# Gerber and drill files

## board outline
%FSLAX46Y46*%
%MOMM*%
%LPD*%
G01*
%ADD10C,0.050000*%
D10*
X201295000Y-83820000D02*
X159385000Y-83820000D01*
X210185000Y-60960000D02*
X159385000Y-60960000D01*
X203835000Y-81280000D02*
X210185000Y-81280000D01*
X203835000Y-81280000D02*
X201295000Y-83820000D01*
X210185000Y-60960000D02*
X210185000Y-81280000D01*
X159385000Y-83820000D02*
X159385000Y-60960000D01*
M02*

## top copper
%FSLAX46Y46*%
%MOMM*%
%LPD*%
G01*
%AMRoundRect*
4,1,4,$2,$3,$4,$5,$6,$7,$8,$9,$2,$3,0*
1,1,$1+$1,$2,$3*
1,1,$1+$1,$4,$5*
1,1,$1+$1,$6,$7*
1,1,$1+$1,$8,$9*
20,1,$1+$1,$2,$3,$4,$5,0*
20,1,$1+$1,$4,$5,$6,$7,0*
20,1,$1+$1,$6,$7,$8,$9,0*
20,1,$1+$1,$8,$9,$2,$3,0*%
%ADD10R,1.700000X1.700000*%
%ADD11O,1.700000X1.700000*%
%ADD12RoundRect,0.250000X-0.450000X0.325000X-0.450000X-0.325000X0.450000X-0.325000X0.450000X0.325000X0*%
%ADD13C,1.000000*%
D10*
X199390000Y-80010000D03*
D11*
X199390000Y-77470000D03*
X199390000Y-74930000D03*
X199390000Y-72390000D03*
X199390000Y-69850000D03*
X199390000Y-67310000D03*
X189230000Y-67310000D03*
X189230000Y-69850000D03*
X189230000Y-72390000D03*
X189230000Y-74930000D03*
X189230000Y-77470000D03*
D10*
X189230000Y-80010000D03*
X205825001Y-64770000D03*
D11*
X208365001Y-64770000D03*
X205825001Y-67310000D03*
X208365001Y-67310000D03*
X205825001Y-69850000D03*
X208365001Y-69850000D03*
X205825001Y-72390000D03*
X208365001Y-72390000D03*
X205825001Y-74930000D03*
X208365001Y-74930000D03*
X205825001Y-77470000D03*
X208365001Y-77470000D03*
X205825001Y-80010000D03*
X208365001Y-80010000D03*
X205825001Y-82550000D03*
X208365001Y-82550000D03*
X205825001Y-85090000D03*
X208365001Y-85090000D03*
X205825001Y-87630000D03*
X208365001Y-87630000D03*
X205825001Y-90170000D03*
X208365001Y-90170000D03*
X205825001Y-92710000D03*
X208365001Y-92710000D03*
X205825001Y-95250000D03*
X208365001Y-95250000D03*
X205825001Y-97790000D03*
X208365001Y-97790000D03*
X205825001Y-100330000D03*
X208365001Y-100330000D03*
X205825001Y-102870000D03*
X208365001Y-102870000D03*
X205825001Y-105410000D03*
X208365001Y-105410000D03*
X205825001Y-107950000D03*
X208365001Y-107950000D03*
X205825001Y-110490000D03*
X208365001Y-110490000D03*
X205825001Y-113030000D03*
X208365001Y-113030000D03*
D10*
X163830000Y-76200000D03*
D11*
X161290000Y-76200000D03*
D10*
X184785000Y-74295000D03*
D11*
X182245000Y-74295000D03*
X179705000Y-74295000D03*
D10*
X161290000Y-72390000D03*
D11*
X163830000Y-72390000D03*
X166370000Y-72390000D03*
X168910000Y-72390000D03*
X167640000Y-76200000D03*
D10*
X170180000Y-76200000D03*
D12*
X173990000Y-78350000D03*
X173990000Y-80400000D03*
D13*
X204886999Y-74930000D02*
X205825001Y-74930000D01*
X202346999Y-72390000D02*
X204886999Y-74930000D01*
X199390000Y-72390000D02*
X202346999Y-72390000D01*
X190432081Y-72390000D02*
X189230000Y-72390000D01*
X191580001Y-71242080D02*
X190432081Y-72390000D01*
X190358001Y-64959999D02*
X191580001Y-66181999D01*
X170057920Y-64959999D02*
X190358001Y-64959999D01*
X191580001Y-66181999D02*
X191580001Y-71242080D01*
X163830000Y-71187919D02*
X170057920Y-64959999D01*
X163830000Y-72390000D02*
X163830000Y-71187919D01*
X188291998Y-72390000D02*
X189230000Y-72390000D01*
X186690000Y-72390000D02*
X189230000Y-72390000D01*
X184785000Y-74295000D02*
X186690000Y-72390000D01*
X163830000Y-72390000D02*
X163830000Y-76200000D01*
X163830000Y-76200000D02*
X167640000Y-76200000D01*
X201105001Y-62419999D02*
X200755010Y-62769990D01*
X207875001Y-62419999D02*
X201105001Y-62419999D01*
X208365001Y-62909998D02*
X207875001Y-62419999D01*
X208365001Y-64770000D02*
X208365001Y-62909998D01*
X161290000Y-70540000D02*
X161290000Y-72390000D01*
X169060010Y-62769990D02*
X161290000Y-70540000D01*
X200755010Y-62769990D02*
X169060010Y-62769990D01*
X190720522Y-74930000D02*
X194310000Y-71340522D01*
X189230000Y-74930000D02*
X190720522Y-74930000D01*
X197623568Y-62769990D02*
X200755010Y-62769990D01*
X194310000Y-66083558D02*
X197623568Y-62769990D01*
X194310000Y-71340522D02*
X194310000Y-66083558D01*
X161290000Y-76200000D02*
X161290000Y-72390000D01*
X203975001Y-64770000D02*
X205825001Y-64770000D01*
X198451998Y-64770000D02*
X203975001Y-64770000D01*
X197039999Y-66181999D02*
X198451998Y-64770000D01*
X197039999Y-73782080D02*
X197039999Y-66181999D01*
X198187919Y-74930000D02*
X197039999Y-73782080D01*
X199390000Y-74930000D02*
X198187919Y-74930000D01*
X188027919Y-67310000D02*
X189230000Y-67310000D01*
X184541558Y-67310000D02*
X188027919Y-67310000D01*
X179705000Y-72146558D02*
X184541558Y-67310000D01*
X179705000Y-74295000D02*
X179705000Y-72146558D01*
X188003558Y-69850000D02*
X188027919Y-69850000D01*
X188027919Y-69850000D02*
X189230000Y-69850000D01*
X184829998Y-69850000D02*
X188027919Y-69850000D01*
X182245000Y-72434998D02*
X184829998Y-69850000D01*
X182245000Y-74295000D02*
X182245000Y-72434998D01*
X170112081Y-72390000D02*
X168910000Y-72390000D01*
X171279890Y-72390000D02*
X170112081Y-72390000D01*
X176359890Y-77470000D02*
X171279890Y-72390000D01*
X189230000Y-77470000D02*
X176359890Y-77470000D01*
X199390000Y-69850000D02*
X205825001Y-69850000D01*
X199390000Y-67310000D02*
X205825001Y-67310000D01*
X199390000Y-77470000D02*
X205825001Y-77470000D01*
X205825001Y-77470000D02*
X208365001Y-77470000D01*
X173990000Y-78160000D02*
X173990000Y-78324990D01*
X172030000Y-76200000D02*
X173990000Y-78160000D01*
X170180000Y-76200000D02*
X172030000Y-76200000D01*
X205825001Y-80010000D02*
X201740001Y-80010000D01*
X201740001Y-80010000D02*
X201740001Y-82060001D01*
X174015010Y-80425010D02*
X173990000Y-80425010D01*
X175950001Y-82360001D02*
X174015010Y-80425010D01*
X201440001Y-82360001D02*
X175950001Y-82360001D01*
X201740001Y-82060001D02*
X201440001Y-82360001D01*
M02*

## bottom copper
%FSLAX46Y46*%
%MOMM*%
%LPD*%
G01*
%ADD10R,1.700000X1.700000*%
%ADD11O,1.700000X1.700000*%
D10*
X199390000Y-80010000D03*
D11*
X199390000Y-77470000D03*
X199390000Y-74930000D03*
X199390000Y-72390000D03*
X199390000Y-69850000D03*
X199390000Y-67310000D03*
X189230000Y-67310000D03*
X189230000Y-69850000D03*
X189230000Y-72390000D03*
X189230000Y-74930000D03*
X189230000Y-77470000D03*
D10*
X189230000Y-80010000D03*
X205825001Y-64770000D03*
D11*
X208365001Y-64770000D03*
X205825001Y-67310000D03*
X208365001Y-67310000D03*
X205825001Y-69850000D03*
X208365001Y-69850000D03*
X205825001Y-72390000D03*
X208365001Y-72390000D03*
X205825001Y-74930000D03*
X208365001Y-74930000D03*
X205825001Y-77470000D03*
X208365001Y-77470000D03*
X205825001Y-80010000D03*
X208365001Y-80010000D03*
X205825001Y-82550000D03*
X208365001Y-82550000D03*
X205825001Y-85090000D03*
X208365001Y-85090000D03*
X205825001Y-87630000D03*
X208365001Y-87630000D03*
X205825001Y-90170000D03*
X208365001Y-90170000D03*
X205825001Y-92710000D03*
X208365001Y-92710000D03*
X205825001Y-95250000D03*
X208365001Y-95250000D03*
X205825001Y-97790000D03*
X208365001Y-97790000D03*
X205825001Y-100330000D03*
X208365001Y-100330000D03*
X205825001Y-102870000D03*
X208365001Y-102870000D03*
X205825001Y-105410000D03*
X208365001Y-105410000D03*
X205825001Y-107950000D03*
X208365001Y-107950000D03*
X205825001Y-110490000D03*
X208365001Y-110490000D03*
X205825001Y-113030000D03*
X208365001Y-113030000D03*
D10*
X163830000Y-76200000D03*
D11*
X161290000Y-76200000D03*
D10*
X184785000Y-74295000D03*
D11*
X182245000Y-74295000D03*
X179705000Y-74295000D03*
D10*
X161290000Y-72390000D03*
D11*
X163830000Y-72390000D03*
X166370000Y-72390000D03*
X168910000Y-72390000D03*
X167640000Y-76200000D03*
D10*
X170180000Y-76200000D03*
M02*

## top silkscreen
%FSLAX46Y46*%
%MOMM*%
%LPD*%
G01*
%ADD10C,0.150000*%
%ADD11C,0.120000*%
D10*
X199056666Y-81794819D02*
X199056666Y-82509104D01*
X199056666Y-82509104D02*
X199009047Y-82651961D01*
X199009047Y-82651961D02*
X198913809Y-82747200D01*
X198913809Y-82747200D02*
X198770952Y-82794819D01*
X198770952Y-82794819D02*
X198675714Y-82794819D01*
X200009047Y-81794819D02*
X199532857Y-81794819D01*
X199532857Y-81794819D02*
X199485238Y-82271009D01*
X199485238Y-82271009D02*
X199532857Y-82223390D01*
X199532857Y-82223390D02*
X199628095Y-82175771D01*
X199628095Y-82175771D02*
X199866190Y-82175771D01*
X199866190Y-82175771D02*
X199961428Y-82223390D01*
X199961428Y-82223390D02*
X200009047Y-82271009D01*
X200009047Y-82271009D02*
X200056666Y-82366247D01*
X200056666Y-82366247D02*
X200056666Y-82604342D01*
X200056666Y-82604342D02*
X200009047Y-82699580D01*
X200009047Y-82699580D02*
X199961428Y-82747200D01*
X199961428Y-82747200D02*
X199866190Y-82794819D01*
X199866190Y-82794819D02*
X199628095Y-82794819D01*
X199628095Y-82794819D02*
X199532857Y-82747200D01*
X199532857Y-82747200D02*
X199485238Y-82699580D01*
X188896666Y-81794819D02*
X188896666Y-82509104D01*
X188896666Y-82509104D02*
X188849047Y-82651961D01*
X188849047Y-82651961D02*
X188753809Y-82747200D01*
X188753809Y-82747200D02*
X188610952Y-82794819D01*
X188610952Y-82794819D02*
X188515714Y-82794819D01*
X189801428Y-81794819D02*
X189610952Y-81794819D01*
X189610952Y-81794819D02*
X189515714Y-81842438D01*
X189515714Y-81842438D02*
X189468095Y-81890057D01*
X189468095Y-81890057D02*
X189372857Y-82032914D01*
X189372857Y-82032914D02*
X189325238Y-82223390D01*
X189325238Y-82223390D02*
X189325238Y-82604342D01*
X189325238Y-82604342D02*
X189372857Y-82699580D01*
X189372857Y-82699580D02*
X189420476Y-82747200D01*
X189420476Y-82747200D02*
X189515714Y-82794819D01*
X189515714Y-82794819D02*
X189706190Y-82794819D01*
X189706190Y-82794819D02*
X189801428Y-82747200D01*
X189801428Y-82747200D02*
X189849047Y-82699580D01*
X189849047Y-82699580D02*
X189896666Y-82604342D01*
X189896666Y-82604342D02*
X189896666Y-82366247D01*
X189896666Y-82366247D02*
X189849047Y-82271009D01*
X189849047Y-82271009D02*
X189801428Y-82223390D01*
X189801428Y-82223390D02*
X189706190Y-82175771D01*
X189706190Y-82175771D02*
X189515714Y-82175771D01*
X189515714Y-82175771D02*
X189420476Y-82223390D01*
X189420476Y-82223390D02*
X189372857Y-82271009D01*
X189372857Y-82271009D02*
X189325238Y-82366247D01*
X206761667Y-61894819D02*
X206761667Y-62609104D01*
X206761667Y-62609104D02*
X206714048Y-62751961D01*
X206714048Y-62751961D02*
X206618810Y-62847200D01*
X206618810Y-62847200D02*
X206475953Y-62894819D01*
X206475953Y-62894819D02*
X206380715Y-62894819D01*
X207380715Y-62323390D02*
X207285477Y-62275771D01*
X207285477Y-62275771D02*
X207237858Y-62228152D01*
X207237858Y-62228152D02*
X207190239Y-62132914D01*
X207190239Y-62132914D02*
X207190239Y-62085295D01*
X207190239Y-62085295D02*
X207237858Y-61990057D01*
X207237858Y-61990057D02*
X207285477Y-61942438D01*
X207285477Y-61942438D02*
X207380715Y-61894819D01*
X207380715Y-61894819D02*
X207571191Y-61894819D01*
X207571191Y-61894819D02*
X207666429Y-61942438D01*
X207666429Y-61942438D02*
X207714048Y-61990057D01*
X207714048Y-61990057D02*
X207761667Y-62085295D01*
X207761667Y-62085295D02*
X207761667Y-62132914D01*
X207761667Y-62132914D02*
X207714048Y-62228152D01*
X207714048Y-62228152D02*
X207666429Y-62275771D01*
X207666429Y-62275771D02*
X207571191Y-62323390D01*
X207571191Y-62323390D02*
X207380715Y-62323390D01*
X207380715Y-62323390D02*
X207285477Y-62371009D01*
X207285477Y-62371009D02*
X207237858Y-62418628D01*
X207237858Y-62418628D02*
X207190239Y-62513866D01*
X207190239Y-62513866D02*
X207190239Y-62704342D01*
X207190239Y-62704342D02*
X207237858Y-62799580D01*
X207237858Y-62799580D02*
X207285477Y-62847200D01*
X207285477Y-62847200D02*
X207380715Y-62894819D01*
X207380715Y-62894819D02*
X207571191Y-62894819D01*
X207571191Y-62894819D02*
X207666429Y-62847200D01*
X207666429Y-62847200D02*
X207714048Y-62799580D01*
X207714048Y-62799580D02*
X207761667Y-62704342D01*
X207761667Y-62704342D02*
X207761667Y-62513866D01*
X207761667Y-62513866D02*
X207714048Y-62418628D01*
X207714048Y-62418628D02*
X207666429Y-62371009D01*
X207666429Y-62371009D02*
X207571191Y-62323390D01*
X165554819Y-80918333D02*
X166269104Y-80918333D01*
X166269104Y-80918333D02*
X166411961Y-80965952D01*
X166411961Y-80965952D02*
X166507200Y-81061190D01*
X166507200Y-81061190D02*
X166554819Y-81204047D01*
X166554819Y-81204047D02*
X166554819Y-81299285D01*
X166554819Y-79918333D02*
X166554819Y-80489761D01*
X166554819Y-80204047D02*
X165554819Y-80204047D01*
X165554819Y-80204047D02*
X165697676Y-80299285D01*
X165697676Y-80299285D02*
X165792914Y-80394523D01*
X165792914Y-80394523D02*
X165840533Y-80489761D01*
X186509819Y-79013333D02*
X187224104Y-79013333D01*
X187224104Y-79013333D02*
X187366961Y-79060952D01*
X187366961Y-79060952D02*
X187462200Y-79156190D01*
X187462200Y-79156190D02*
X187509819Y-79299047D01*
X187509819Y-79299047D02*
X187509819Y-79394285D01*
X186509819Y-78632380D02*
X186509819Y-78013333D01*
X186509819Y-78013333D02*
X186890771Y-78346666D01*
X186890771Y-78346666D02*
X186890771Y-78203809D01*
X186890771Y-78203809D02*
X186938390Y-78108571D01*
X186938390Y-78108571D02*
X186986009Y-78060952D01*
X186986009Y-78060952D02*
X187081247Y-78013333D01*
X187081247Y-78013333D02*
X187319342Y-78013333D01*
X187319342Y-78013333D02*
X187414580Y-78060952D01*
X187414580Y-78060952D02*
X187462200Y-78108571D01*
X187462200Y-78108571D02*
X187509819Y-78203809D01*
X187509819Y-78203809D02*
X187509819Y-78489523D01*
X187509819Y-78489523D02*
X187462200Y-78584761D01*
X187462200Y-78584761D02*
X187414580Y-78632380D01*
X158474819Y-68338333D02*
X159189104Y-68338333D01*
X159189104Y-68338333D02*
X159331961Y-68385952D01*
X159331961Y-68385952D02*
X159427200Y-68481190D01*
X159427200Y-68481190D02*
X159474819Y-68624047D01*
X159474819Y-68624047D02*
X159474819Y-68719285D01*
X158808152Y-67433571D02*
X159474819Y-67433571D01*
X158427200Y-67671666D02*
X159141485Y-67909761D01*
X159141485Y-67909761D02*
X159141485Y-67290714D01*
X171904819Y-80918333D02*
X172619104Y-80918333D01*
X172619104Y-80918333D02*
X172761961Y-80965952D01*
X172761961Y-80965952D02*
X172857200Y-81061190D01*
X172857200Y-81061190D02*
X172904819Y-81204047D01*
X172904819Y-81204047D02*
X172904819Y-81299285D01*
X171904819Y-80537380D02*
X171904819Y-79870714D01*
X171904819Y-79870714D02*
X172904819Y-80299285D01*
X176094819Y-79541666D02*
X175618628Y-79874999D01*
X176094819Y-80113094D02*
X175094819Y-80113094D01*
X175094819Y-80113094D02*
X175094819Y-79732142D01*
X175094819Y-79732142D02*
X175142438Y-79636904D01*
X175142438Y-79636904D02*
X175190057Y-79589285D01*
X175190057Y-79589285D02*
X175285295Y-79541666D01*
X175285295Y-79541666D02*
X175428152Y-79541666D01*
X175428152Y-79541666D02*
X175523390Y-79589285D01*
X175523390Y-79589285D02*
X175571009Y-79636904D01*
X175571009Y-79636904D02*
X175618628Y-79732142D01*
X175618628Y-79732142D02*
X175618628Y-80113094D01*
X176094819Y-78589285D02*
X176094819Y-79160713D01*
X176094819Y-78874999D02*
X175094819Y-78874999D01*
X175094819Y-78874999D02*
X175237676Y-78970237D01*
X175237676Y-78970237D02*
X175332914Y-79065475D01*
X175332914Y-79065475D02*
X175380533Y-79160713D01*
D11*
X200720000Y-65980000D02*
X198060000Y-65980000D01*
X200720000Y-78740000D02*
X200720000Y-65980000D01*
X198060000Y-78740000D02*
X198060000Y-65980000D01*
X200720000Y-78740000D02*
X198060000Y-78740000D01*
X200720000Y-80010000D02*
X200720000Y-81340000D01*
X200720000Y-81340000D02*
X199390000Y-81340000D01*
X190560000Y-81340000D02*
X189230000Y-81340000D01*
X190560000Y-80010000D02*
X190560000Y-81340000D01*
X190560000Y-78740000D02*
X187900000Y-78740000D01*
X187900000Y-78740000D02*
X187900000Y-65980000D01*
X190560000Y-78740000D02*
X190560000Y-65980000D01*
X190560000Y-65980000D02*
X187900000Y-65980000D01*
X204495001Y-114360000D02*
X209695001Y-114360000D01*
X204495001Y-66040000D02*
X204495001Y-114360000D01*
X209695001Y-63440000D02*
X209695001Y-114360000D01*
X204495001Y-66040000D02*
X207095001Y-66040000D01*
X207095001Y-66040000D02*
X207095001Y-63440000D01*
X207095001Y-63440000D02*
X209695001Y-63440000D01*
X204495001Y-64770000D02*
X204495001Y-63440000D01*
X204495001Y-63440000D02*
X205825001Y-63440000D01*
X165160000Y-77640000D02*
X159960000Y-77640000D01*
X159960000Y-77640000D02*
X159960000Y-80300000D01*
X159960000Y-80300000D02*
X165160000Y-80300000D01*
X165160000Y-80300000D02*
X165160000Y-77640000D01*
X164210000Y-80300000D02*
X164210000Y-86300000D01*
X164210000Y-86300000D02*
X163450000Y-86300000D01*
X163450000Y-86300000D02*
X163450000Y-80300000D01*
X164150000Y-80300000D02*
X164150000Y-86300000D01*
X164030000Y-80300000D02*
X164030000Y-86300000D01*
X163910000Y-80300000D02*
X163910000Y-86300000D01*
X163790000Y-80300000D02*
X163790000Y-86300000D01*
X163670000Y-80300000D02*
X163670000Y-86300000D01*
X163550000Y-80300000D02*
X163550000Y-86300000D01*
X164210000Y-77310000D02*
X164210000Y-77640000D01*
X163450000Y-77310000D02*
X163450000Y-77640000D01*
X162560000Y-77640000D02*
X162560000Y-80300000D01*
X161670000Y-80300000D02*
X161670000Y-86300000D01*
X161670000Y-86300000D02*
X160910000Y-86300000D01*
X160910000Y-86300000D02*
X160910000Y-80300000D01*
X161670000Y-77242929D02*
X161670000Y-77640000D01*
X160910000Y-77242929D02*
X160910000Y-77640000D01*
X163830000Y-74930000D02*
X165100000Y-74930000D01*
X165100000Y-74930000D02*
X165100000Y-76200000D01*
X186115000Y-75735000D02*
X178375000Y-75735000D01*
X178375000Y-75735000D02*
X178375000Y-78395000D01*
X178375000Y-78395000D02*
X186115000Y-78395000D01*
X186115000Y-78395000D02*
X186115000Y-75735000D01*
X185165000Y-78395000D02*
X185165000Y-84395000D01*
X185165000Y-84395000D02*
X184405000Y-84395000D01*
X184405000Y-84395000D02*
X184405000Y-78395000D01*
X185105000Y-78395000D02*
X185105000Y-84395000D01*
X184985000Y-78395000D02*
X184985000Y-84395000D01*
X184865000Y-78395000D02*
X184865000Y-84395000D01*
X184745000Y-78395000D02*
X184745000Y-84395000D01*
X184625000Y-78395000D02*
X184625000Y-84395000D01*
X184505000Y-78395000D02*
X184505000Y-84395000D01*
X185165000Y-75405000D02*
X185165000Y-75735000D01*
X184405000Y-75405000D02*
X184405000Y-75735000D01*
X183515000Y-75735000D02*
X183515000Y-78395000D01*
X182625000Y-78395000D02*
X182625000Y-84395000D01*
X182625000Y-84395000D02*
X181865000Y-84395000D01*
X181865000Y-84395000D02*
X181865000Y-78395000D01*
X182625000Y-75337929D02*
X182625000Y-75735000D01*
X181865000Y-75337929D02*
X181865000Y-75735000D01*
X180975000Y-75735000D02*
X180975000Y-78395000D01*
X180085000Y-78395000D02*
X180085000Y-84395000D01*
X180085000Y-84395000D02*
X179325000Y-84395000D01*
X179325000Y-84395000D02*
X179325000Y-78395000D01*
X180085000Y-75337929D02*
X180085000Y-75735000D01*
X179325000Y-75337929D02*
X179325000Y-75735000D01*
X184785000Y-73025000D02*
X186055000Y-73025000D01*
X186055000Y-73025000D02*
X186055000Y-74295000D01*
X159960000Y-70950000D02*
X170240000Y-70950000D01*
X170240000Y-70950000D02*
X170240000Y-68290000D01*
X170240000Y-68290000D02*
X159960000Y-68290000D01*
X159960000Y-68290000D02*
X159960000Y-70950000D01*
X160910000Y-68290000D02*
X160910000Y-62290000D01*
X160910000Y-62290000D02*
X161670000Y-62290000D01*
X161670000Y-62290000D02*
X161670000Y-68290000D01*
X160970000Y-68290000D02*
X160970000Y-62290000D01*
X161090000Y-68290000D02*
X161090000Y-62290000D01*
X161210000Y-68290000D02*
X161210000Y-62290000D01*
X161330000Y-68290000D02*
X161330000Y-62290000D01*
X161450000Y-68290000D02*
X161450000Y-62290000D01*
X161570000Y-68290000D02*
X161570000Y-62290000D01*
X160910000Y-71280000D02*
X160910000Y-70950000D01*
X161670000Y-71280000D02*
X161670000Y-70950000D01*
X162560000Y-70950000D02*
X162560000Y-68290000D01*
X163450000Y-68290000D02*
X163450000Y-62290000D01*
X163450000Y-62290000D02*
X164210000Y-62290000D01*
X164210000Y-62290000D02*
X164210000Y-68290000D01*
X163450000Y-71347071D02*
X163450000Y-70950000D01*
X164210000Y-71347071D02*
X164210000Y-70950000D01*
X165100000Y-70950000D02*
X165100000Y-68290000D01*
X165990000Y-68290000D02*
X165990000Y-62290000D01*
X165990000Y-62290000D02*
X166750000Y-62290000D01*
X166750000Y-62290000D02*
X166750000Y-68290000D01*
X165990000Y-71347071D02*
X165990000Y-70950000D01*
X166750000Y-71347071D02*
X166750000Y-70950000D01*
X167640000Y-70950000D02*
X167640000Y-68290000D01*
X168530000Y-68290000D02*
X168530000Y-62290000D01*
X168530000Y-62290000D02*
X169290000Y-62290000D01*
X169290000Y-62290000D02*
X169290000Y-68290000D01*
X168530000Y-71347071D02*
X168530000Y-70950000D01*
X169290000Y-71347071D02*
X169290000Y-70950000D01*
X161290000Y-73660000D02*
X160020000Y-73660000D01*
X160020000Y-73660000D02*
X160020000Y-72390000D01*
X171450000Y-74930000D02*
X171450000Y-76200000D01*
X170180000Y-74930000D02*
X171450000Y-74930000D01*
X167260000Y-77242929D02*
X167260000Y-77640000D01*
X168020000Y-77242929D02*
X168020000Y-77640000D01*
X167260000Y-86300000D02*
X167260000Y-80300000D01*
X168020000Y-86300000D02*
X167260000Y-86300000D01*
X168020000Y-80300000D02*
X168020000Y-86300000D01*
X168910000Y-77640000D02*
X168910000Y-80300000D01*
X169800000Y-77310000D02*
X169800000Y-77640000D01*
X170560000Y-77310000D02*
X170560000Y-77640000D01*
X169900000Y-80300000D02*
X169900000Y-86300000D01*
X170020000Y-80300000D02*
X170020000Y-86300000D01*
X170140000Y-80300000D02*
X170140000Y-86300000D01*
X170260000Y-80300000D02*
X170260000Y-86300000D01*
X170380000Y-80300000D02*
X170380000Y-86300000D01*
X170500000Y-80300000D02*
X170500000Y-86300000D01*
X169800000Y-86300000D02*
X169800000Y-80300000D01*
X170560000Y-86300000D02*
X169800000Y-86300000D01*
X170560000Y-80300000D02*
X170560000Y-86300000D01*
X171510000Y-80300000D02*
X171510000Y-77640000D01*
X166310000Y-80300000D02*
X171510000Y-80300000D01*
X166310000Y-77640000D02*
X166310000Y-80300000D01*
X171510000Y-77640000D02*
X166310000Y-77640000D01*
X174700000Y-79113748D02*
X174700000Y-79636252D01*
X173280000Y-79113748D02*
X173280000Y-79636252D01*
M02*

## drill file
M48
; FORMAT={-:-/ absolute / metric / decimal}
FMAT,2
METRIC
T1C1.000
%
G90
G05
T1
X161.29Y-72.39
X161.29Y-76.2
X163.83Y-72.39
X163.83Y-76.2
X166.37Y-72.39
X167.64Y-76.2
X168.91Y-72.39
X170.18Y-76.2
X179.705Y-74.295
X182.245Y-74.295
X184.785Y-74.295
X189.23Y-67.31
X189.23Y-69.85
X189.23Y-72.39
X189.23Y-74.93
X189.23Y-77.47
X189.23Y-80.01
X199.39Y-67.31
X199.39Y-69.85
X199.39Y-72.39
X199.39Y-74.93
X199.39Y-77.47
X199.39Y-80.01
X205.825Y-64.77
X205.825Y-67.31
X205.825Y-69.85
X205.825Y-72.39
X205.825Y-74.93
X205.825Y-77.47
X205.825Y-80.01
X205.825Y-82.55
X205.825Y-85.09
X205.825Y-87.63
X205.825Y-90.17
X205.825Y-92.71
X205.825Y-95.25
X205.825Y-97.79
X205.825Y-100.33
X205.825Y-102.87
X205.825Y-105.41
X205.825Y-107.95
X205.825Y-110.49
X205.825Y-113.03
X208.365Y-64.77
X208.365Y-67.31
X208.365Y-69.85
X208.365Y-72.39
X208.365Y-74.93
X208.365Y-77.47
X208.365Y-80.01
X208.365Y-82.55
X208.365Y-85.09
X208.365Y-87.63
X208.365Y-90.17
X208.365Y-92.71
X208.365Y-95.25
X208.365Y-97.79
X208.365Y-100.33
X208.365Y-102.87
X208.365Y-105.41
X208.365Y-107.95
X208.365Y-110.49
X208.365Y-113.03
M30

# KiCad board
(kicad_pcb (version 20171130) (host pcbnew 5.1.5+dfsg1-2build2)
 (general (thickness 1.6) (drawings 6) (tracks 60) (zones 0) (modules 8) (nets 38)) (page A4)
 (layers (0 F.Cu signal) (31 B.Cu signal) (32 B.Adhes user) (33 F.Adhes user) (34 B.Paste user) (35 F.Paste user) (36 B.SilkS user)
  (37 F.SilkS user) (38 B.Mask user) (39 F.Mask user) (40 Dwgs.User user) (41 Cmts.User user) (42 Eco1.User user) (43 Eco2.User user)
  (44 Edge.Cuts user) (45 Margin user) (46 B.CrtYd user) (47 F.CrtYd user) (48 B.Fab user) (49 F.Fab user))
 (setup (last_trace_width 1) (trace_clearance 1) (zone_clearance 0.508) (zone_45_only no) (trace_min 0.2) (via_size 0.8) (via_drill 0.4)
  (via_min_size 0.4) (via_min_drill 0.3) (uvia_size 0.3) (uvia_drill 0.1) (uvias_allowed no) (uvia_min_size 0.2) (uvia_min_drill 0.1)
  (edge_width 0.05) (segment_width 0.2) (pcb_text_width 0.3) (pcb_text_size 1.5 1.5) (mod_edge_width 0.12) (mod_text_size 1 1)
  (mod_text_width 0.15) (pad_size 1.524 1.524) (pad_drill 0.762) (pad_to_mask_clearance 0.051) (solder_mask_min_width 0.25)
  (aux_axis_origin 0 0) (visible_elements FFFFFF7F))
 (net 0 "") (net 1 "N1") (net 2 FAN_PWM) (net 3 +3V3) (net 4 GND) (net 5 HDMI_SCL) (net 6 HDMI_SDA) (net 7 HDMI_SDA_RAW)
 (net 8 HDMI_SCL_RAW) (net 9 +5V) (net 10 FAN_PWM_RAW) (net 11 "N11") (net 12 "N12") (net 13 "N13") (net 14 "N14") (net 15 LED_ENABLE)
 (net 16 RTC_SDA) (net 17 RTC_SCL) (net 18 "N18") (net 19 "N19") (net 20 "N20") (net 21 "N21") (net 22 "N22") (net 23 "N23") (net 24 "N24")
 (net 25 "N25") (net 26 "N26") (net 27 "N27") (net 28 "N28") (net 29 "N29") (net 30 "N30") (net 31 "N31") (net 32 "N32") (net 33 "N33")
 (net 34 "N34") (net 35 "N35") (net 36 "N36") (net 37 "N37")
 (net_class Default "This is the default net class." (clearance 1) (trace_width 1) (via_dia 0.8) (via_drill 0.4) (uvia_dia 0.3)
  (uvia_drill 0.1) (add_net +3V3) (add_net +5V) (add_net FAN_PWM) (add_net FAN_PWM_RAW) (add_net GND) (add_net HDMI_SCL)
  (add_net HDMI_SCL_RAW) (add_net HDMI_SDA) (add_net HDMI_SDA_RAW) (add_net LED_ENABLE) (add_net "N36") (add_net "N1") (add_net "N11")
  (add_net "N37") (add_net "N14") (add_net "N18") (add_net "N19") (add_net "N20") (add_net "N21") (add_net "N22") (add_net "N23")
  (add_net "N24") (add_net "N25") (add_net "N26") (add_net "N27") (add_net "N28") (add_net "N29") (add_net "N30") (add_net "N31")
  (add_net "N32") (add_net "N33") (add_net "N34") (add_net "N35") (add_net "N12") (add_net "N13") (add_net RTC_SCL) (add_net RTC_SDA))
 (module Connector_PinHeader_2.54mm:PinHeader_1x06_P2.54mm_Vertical (layer F.Cu) (at 199.39 80.01 180)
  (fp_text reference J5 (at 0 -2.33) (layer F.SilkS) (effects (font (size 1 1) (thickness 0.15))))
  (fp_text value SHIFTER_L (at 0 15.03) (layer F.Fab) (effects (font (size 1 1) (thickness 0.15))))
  (fp_line (start -1.33 14.03) (end 1.33 14.03) (layer F.SilkS) (width 0.12))
  (fp_line (start -1.33 1.27) (end -1.33 14.03) (layer F.SilkS) (width 0.12))
  (fp_line (start 1.33 1.27) (end 1.33 14.03) (layer F.SilkS) (width 0.12))
  (fp_line (start -1.33 1.27) (end 1.33 1.27) (layer F.SilkS) (width 0.12))
  (fp_line (start -1.33 0) (end -1.33 -1.33) (layer F.SilkS) (width 0.12))
  (fp_line (start -1.33 -1.33) (end 0 -1.33) (layer F.SilkS) (width 0.12))
  (pad 1 thru_hole rect (at 0 0 180) (size 1.7 1.7) (drill 1) (layers *.Cu *.Mask) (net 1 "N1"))
  (pad 2 thru_hole oval (at 0 2.54 180) (size 1.7 1.7) (drill 1) (layers *.Cu *.Mask) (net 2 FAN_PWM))
  (pad 3 thru_hole oval (at 0 5.08 180) (size 1.7 1.7) (drill 1) (layers *.Cu *.Mask) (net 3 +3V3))
  (pad 4 thru_hole oval (at 0 7.62 180) (size 1.7 1.7) (drill 1) (layers *.Cu *.Mask) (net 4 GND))
  (pad 5 thru_hole oval (at 0 10.16 180) (size 1.7 1.7) (drill 1) (layers *.Cu *.Mask) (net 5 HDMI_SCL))
  (pad 6 thru_hole oval (at 0 12.7 180) (size 1.7 1.7) (drill 1) (layers *.Cu *.Mask) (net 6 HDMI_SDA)))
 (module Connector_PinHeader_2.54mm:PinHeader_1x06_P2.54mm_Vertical (layer F.Cu) (at 189.23 80.01 180)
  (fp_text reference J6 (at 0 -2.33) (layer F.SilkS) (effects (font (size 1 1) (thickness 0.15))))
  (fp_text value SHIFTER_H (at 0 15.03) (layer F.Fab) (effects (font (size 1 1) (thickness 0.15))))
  (fp_line (start -1.33 -1.33) (end 0 -1.33) (layer F.SilkS) (width 0.12))
  (fp_line (start -1.33 0) (end -1.33 -1.33) (layer F.SilkS) (width 0.12))
  (fp_line (start -1.33 1.27) (end 1.33 1.27) (layer F.SilkS) (width 0.12))
  (fp_line (start 1.33 1.27) (end 1.33 14.03) (layer F.SilkS) (width 0.12))
  (fp_line (start -1.33 1.27) (end -1.33 14.03) (layer F.SilkS) (width 0.12))
  (fp_line (start -1.33 14.03) (end 1.33 14.03) (layer F.SilkS) (width 0.12))
  (pad 6 thru_hole oval (at 0 12.7 180) (size 1.7 1.7) (drill 1) (layers *.Cu *.Mask) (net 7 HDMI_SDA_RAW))
  (pad 5 thru_hole oval (at 0 10.16 180) (size 1.7 1.7) (drill 1) (layers *.Cu *.Mask) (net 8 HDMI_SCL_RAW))
  (pad 4 thru_hole oval (at 0 7.62 180) (size 1.7 1.7) (drill 1) (layers *.Cu *.Mask) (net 4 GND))
  (pad 3 thru_hole oval (at 0 5.08 180) (size 1.7 1.7) (drill 1) (layers *.Cu *.Mask) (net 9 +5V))
  (pad 2 thru_hole oval (at 0 2.54 180) (size 1.7 1.7) (drill 1) (layers *.Cu *.Mask) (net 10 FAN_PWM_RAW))
  (pad 1 thru_hole rect (at 0 0 180) (size 1.7 1.7) (drill 1) (layers *.Cu *.Mask) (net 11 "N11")))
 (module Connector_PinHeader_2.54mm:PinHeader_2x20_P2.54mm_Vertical (layer F.Cu) (at 205.825001 64.77)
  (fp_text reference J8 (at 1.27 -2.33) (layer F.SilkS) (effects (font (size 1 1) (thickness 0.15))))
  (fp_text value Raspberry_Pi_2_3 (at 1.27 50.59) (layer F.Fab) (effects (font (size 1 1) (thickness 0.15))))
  (fp_line (start -1.33 49.59) (end 3.87 49.59) (layer F.SilkS) (width 0.12))
  (fp_line (start -1.33 1.27) (end -1.33 49.59) (layer F.SilkS) (width 0.12))
  (fp_line (start 3.87 -1.33) (end 3.87 49.59) (layer F.SilkS) (width 0.12))
  (fp_line (start -1.33 1.27) (end 1.27 1.27) (layer F.SilkS) (width 0.12))
  (fp_line (start 1.27 1.27) (end 1.27 -1.33) (layer F.SilkS) (width 0.12))
  (fp_line (start 1.27 -1.33) (end 3.87 -1.33) (layer F.SilkS) (width 0.12))
  (fp_line (start -1.33 0) (end -1.33 -1.33) (layer F.SilkS) (width 0.12))
  (fp_line (start -1.33 -1.33) (end 0 -1.33) (layer F.SilkS) (width 0.12))
  (pad 1 thru_hole rect (at 0 0) (size 1.7 1.7) (drill 1) (layers *.Cu *.Mask) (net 3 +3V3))
  (pad 2 thru_hole oval (at 2.54 0) (size 1.7 1.7) (drill 1) (layers *.Cu *.Mask) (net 9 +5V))
  (pad 3 thru_hole oval (at 0 2.54) (size 1.7 1.7) (drill 1) (layers *.Cu *.Mask) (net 6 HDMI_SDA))
  (pad 4 thru_hole oval (at 2.54 2.54) (size 1.7 1.7) (drill 1) (layers *.Cu *.Mask) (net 9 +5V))
  (pad 5 thru_hole oval (at 0 5.08) (size 1.7 1.7) (drill 1) (layers *.Cu *.Mask) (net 5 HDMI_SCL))
  (pad 6 thru_hole oval (at 2.54 5.08) (size 1.7 1.7) (drill 1) (layers *.Cu *.Mask) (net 4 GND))
  (pad 7 thru_hole oval (at 0 7.62) (size 1.7 1.7) (drill 1) (layers *.Cu *.Mask) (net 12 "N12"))
  (pad 8 thru_hole oval (at 2.54 7.62) (size 1.7 1.7) (drill 1) (layers *.Cu *.Mask) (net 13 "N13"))
  (pad 9 thru_hole oval (at 0 10.16) (size 1.7 1.7) (drill 1) (layers *.Cu *.Mask) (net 4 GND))
  (pad 10 thru_hole oval (at 2.54 10.16) (size 1.7 1.7) (drill 1) (layers *.Cu *.Mask) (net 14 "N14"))
  (pad 11 thru_hole oval (at 0 12.7) (size 1.7 1.7) (drill 1) (layers *.Cu *.Mask) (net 2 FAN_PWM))
  (pad 12 thru_hole oval (at 2.54 12.7) (size 1.7 1.7) (drill 1) (layers *.Cu *.Mask) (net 2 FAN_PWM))
  (pad 13 thru_hole oval (at 0 15.24) (size 1.7 1.7) (drill 1) (layers *.Cu *.Mask) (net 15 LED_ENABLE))
  (pad 14 thru_hole oval (at 2.54 15.24) (size 1.7 1.7) (drill 1) (layers *.Cu *.Mask) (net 4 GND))
  (pad 15 thru_hole oval (at 0 17.78) (size 1.7 1.7) (drill 1) (layers *.Cu *.Mask) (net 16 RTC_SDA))
  (pad 16 thru_hole oval (at 2.54 17.78) (size 1.7 1.7) (drill 1) (layers *.Cu *.Mask) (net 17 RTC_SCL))
  (pad 17 thru_hole oval (at 0 20.32) (size 1.7 1.7) (drill 1) (layers *.Cu *.Mask) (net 3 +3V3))
  (pad 18 thru_hole oval (at 2.54 20.32) (size 1.7 1.7) (drill 1) (layers *.Cu *.Mask) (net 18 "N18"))
  (pad 19 thru_hole oval (at 0 22.86) (size 1.7 1.7) (drill 1) (layers *.Cu *.Mask) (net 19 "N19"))
  (pad 20 thru_hole oval (at 2.54 22.86) (size 1.7 1.7) (drill 1) (layers *.Cu *.Mask) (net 4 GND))
  (pad 21 thru_hole oval (at 0 25.4) (size 1.7 1.7) (drill 1) (layers *.Cu *.Mask) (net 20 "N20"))
  (pad 22 thru_hole oval (at 2.54 25.4) (size 1.7 1.7) (drill 1) (layers *.Cu *.Mask) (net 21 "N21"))
  (pad 23 thru_hole oval (at 0 27.94) (size 1.7 1.7) (drill 1) (layers *.Cu *.Mask) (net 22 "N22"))
  (pad 24 thru_hole oval (at 2.54 27.94) (size 1.7 1.7) (drill 1) (layers *.Cu *.Mask) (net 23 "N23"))
  (pad 25 thru_hole oval (at 0 30.48) (size 1.7 1.7) (drill 1) (layers *.Cu *.Mask) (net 4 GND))
  (pad 26 thru_hole oval (at 2.54 30.48) (size 1.7 1.7) (drill 1) (layers *.Cu *.Mask) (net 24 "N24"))
  (pad 27 thru_hole oval (at 0 33.02) (size 1.7 1.7) (drill 1) (layers *.Cu *.Mask) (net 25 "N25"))
  (pad 28 thru_hole oval (at 2.54 33.02) (size 1.7 1.7) (drill 1) (layers *.Cu *.Mask) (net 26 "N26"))
  (pad 29 thru_hole oval (at 0 35.56) (size 1.7 1.7) (drill 1) (layers *.Cu *.Mask) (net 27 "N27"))
  (pad 30 thru_hole oval (at 2.54 35.56) (size 1.7 1.7) (drill 1) (layers *.Cu *.Mask) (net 4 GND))
  (pad 31 thru_hole oval (at 0 38.1) (size 1.7 1.7) (drill 1) (layers *.Cu *.Mask) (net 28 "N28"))
  (pad 32 thru_hole oval (at 2.54 38.1) (size 1.7 1.7) (drill 1) (layers *.Cu *.Mask) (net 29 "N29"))
  (pad 33 thru_hole oval (at 0 40.64) (size 1.7 1.7) (drill 1) (layers *.Cu *.Mask) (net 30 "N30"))
  (pad 34 thru_hole oval (at 2.54 40.64) (size 1.7 1.7) (drill 1) (layers *.Cu *.Mask) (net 4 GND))
  (pad 35 thru_hole oval (at 0 43.18) (size 1.7 1.7) (drill 1) (layers *.Cu *.Mask) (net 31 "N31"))
  (pad 36 thru_hole oval (at 2.54 43.18) (size 1.7 1.7) (drill 1) (layers *.Cu *.Mask) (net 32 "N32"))
  (pad 37 thru_hole oval (at 0 45.72) (size 1.7 1.7) (drill 1) (layers *.Cu *.Mask) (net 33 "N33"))
  (pad 38 thru_hole oval (at 2.54 45.72) (size 1.7 1.7) (drill 1) (layers *.Cu *.Mask) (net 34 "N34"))
  (pad 39 thru_hole oval (at 0 48.26) (size 1.7 1.7) (drill 1) (layers *.Cu *.Mask) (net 4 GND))
  (pad 40 thru_hole oval (at 2.54 48.26) (size 1.7 1.7) (drill 1) (layers *.Cu *.Mask) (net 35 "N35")))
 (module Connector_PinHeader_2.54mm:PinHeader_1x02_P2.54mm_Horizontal (layer F.Cu) (at 163.83 76.2 270)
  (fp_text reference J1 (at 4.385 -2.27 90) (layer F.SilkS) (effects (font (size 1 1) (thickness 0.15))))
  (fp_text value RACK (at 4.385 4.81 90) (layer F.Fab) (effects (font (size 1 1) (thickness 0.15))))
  (fp_line (start 1.44 -1.33) (end 1.44 3.87) (layer F.SilkS) (width 0.12))
  (fp_line (start 1.44 3.87) (end 4.1 3.87) (layer F.SilkS) (width 0.12))
  (fp_line (start 4.1 3.87) (end 4.1 -1.33) (layer F.SilkS) (width 0.12))
  (fp_line (start 4.1 -1.33) (end 1.44 -1.33) (layer F.SilkS) (width 0.12))
  (fp_line (start 4.1 -0.38) (end 10.1 -0.38) (layer F.SilkS) (width 0.12))
  (fp_line (start 10.1 -0.38) (end 10.1 0.38) (layer F.SilkS) (width 0.12))
  (fp_line (start 10.1 0.38) (end 4.1 0.38) (layer F.SilkS) (width 0.12))
  (fp_line (start 4.1 -0.32) (end 10.1 -0.32) (layer F.SilkS) (width 0.12))
  (fp_line (start 4.1 -0.2) (end 10.1 -0.2) (layer F.SilkS) (width 0.12))
  (fp_line (start 4.1 -0.08) (end 10.1 -0.08) (layer F.SilkS) (width 0.12))
  (fp_line (start 4.1 0.04) (end 10.1 0.04) (layer F.SilkS) (width 0.12))
  (fp_line (start 4.1 0.16) (end 10.1 0.16) (layer F.SilkS) (width 0.12))
  (fp_line (start 4.1 0.28) (end 10.1 0.28) (layer F.SilkS) (width 0.12))
  (fp_line (start 1.11 -0.38) (end 1.44 -0.38) (layer F.SilkS) (width 0.12))
  (fp_line (start 1.11 0.38) (end 1.44 0.38) (layer F.SilkS) (width 0.12))
  (fp_line (start 1.44 1.27) (end 4.1 1.27) (layer F.SilkS) (width 0.12))
  (fp_line (start 4.1 2.16) (end 10.1 2.16) (layer F.SilkS) (width 0.12))
  (fp_line (start 10.1 2.16) (end 10.1 2.92) (layer F.SilkS) (width 0.12))
  (fp_line (start 10.1 2.92) (end 4.1 2.92) (layer F.SilkS) (width 0.12))
  (fp_line (start 1.042929 2.16) (end 1.44 2.16) (layer F.SilkS) (width 0.12))
  (fp_line (start 1.042929 2.92) (end 1.44 2.92) (layer F.SilkS) (width 0.12))
  (fp_line (start -1.27 0) (end -1.27 -1.27) (layer F.SilkS) (width 0.12))
  (fp_line (start -1.27 -1.27) (end 0 -1.27) (layer F.SilkS) (width 0.12))
  (pad 1 thru_hole rect (at 0 0 270) (size 1.7 1.7) (drill 1) (layers *.Cu *.Mask) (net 4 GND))
  (pad 2 thru_hole oval (at 0 2.54 270) (size 1.7 1.7) (drill 1) (layers *.Cu *.Mask) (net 9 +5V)))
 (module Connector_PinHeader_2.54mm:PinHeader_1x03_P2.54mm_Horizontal (layer F.Cu) (at 184.785 74.295 270)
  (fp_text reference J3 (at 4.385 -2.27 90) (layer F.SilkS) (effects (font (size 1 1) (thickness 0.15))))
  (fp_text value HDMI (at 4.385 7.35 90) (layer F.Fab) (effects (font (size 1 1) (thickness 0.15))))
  (fp_line (start 1.44 -1.33) (end 1.44 6.41) (layer F.SilkS) (width 0.12))
  (fp_line (start 1.44 6.41) (end 4.1 6.41) (layer F.SilkS) (width 0.12))
  (fp_line (start 4.1 6.41) (end 4.1 -1.33) (layer F.SilkS) (width 0.12))
  (fp_line (start 4.1 -1.33) (end 1.44 -1.33) (layer F.SilkS) (width 0.12))
  (fp_line (start 4.1 -0.38) (end 10.1 -0.38) (layer F.SilkS) (width 0.12))
  (fp_line (start 10.1 -0.38) (end 10.1 0.38) (layer F.SilkS) (width 0.12))
  (fp_line (start 10.1 0.38) (end 4.1 0.38) (layer F.SilkS) (width 0.12))
  (fp_line (start 4.1 -0.32) (end 10.1 -0.32) (layer F.SilkS) (width 0.12))
  (fp_line (start 4.1 -0.2) (end 10.1 -0.2) (layer F.SilkS) (width 0.12))
  (fp_line (start 4.1 -0.08) (end 10.1 -0.08) (layer F.SilkS) (width 0.12))
  (fp_line (start 4.1 0.04) (end 10.1 0.04) (layer F.SilkS) (width 0.12))
  (fp_line (start 4.1 0.16) (end 10.1 0.16) (layer F.SilkS) (width 0.12))
  (fp_line (start 4.1 0.28) (end 10.1 0.28) (layer F.SilkS) (width 0.12))
  (fp_line (start 1.11 -0.38) (end 1.44 -0.38) (layer F.SilkS) (width 0.12))
  (fp_line (start 1.11 0.38) (end 1.44 0.38) (layer F.SilkS) (width 0.12))
  (fp_line (start 1.44 1.27) (end 4.1 1.27) (layer F.SilkS) (width 0.12))
  (fp_line (start 4.1 2.16) (end 10.1 2.16) (layer F.SilkS) (width 0.12))
  (fp_line (start 10.1 2.16) (end 10.1 2.92) (layer F.SilkS) (width 0.12))
  (fp_line (start 10.1 2.92) (end 4.1 2.92) (layer F.SilkS) (width 0.12))
  (fp_line (start 1.042929 2.16) (end 1.44 2.16) (layer F.SilkS) (width 0.12))
  (fp_line (start 1.042929 2.92) (end 1.44 2.92) (layer F.SilkS) (width 0.12))
  (fp_line (start 1.44 3.81) (end 4.1 3.81) (layer F.SilkS) (width 0.12))
  (fp_line (start 4.1 4.7) (end 10.1 4.7) (layer F.SilkS) (width 0.12))
  (fp_line (start 10.1 4.7) (end 10.1 5.46) (layer F.SilkS) (width 0.12))
  (fp_line (start 10.1 5.46) (end 4.1 5.46) (layer F.SilkS) (width 0.12))
  (fp_line (start 1.042929 4.7) (end 1.44 4.7) (layer F.SilkS) (width 0.12))
  (fp_line (start 1.042929 5.46) (end 1.44 5.46) (layer F.SilkS) (width 0.12))
  (fp_line (start -1.27 0) (end -1.27 -1.27) (layer F.SilkS) (width 0.12))
  (fp_line (start -1.27 -1.27) (end 0 -1.27) (layer F.SilkS) (width 0.12))
  (pad 1 thru_hole rect (at 0 0 270) (size 1.7 1.7) (drill 1) (layers *.Cu *.Mask) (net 4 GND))
  (pad 2 thru_hole oval (at 0 2.54 270) (size 1.7 1.7) (drill 1) (layers *.Cu *.Mask) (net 8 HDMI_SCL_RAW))
  (pad 3 thru_hole oval (at 0 5.08 270) (size 1.7 1.7) (drill 1) (layers *.Cu *.Mask) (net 7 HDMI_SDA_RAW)))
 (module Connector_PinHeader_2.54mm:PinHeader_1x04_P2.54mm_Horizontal (layer F.Cu) (at 161.29 72.39 90)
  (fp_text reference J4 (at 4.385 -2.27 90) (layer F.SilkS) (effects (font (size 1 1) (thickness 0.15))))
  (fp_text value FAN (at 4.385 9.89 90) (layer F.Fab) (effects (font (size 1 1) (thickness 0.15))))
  (fp_line (start 1.44 -1.33) (end 1.44 8.95) (layer F.SilkS) (width 0.12))
  (fp_line (start 1.44 8.95) (end 4.1 8.95) (layer F.SilkS) (width 0.12))
  (fp_line (start 4.1 8.95) (end 4.1 -1.33) (layer F.SilkS) (width 0.12))
  (fp_line (start 4.1 -1.33) (end 1.44 -1.33) (layer F.SilkS) (width 0.12))
  (fp_line (start 4.1 -0.38) (end 10.1 -0.38) (layer F.SilkS) (width 0.12))
  (fp_line (start 10.1 -0.38) (end 10.1 0.38) (layer F.SilkS) (width 0.12))
  (fp_line (start 10.1 0.38) (end 4.1 0.38) (layer F.SilkS) (width 0.12))
  (fp_line (start 4.1 -0.32) (end 10.1 -0.32) (layer F.SilkS) (width 0.12))
  (fp_line (start 4.1 -0.2) (end 10.1 -0.2) (layer F.SilkS) (width 0.12))
  (fp_line (start 4.1 -0.08) (end 10.1 -0.08) (layer F.SilkS) (width 0.12))
  (fp_line (start 4.1 0.04) (end 10.1 0.04) (layer F.SilkS) (width 0.12))
  (fp_line (start 4.1 0.16) (end 10.1 0.16) (layer F.SilkS) (width 0.12))
  (fp_line (start 4.1 0.28) (end 10.1 0.28) (layer F.SilkS) (width 0.12))
  (fp_line (start 1.11 -0.38) (end 1.44 -0.38) (layer F.SilkS) (width 0.12))
  (fp_line (start 1.11 0.38) (end 1.44 0.38) (layer F.SilkS) (width 0.12))
  (fp_line (start 1.44 1.27) (end 4.1 1.27) (layer F.SilkS) (width 0.12))
  (fp_line (start 4.1 2.16) (end 10.1 2.16) (layer F.SilkS) (width 0.12))
  (fp_line (start 10.1 2.16) (end 10.1 2.92) (layer F.SilkS) (width 0.12))
  (fp_line (start 10.1 2.92) (end 4.1 2.92) (layer F.SilkS) (width 0.12))
  (fp_line (start 1.042929 2.16) (end 1.44 2.16) (layer F.SilkS) (width 0.12))
  (fp_line (start 1.042929 2.92) (end 1.44 2.92) (layer F.SilkS) (width 0.12))
  (fp_line (start 1.44 3.81) (end 4.1 3.81) (layer F.SilkS) (width 0.12))
  (fp_line (start 4.1 4.7) (end 10.1 4.7) (layer F.SilkS) (width 0.12))
  (fp_line (start 10.1 4.7) (end 10.1 5.46) (layer F.SilkS) (width 0.12))
  (fp_line (start 10.1 5.46) (end 4.1 5.46) (layer F.SilkS) (width 0.12))
  (fp_line (start 1.042929 4.7) (end 1.44 4.7) (layer F.SilkS) (width 0.12))
  (fp_line (start 1.042929 5.46) (end 1.44 5.46) (layer F.SilkS) (width 0.12))
  (fp_line (start 1.44 6.35) (end 4.1 6.35) (layer F.SilkS) (width 0.12))
  (fp_line (start 4.1 7.24) (end 10.1 7.24) (layer F.SilkS) (width 0.12))
  (fp_line (start 10.1 7.24) (end 10.1 8) (layer F.SilkS) (width 0.12))
  (fp_line (start 10.1 8) (end 4.1 8) (layer F.SilkS) (width 0.12))
  (fp_line (start 1.042929 7.24) (end 1.44 7.24) (layer F.SilkS) (width 0.12))
  (fp_line (start 1.042929 8) (end 1.44 8) (layer F.SilkS) (width 0.12))
  (fp_line (start -1.27 0) (end -1.27 -1.27) (layer F.SilkS) (width 0.12))
  (fp_line (start -1.27 -1.27) (end 0 -1.27) (layer F.SilkS) (width 0.12))
  (pad 1 thru_hole rect (at 0 0 90) (size 1.7 1.7) (drill 1) (layers *.Cu *.Mask) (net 9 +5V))
  (pad 2 thru_hole oval (at 0 2.54 90) (size 1.7 1.7) (drill 1) (layers *.Cu *.Mask) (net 4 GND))
  (pad 3 thru_hole oval (at 0 5.08 90) (size 1.7 1.7) (drill 1) (layers *.Cu *.Mask) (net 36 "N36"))
  (pad 4 thru_hole oval (at 0 7.62 90) (size 1.7 1.7) (drill 1) (layers *.Cu *.Mask) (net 10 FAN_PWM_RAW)))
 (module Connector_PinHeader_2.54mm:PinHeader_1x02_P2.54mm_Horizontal (layer F.Cu) (at 170.18 76.2 270)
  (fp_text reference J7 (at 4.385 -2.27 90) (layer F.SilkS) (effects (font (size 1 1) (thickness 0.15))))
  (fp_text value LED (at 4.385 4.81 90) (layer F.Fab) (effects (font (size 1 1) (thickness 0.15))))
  (fp_line (start -1.27 -1.27) (end 0 -1.27) (layer F.SilkS) (width 0.12))
  (fp_line (start -1.27 0) (end -1.27 -1.27) (layer F.SilkS) (width 0.12))
  (fp_line (start 1.042929 2.92) (end 1.44 2.92) (layer F.SilkS) (width 0.12))
  (fp_line (start 1.042929 2.16) (end 1.44 2.16) (layer F.SilkS) (width 0.12))
  (fp_line (start 10.1 2.92) (end 4.1 2.92) (layer F.SilkS) (width 0.12))
  (fp_line (start 10.1 2.16) (end 10.1 2.92) (layer F.SilkS) (width 0.12))
  (fp_line (start 4.1 2.16) (end 10.1 2.16) (layer F.SilkS) (width 0.12))
  (fp_line (start 1.44 1.27) (end 4.1 1.27) (layer F.SilkS) (width 0.12))
  (fp_line (start 1.11 0.38) (end 1.44 0.38) (layer F.SilkS) (width 0.12))
  (fp_line (start 1.11 -0.38) (end 1.44 -0.38) (layer F.SilkS) (width 0.12))
  (fp_line (start 4.1 0.28) (end 10.1 0.28) (layer F.SilkS) (width 0.12))
  (fp_line (start 4.1 0.16) (end 10.1 0.16) (layer F.SilkS) (width 0.12))
  (fp_line (start 4.1 0.04) (end 10.1 0.04) (layer F.SilkS) (width 0.12))
  (fp_line (start 4.1 -0.08) (end 10.1 -0.08) (layer F.SilkS) (width 0.12))
  (fp_line (start 4.1 -0.2) (end 10.1 -0.2) (layer F.SilkS) (width 0.12))
  (fp_line (start 4.1 -0.32) (end 10.1 -0.32) (layer F.SilkS) (width 0.12))
  (fp_line (start 10.1 0.38) (end 4.1 0.38) (layer F.SilkS) (width 0.12))
  (fp_line (start 10.1 -0.38) (end 10.1 0.38) (layer F.SilkS) (width 0.12))
  (fp_line (start 4.1 -0.38) (end 10.1 -0.38) (layer F.SilkS) (width 0.12))
  (fp_line (start 4.1 -1.33) (end 1.44 -1.33) (layer F.SilkS) (width 0.12))
  (fp_line (start 4.1 3.87) (end 4.1 -1.33) (layer F.SilkS) (width 0.12))
  (fp_line (start 1.44 3.87) (end 4.1 3.87) (layer F.SilkS) (width 0.12))
  (fp_line (start 1.44 -1.33) (end 1.44 3.87) (layer F.SilkS) (width 0.12))
  (pad 2 thru_hole oval (at 0 2.54 270) (size 1.7 1.7) (drill 1) (layers *.Cu *.Mask) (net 4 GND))
  (pad 1 thru_hole rect (at 0 0 270) (size 1.7 1.7) (drill 1) (layers *.Cu *.Mask) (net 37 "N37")))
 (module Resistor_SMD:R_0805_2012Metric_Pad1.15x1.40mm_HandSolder (layer F.Cu) (at 173.99 79.375 270)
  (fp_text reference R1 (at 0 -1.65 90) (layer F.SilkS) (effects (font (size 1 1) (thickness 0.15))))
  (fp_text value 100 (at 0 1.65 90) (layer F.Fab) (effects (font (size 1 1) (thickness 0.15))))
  (fp_line (start -0.261252 -0.71) (end 0.261252 -0.71) (layer F.SilkS) (width 0.12))
  (fp_line (start -0.261252 0.71) (end 0.261252 0.71) (layer F.SilkS) (width 0.12))
  (pad 1 smd roundrect (at -1.025 0 270) (size 1.15 1.4) (layers F.Cu F.Paste F.Mask) (roundrect_rratio 0.217391) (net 37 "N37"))
  (pad 2 smd roundrect (at 1.025 0 270) (size 1.15 1.4) (layers F.Cu F.Paste F.Mask) (roundrect_rratio 0.217391) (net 15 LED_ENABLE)))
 (gr_line (start 201.295 83.82) (end 159.385 83.82) (layer Edge.Cuts) (width 0.05))
 (gr_line (start 210.185 60.96) (end 159.385 60.96) (layer Edge.Cuts) (width 0.05))
 (gr_line (start 203.835 81.28) (end 210.185 81.28) (layer Edge.Cuts) (width 0.05))
 (gr_line (start 203.835 81.28) (end 201.295 83.82) (layer Edge.Cuts) (width 0.05))
 (gr_line (start 210.185 60.96) (end 210.185 81.28) (layer Edge.Cuts) (width 0.05))
 (gr_line (start 159.385 83.82) (end 159.385 60.96) (layer Edge.Cuts) (width 0.05))
 (segment (start 204.886999 74.93) (end 205.825001 74.93) (width 1) (layer F.Cu) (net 4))
 (segment (start 202.346999 72.39) (end 204.886999 74.93) (width 1) (layer F.Cu) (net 4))
 (segment (start 199.39 72.39) (end 202.346999 72.39) (width 1) (layer F.Cu) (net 4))
 (segment (start 190.432081 72.39) (end 189.23 72.39) (width 1) (layer F.Cu) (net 4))
 (segment (start 191.580001 71.24208) (end 190.432081 72.39) (width 1) (layer F.Cu) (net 4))
 (segment (start 190.358001 64.959999) (end 191.580001 66.181999) (width 1) (layer F.Cu) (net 4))
 (segment (start 170.05792 64.959999) (end 190.358001 64.959999) (width 1) (layer F.Cu) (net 4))
 (segment (start 191.580001 66.181999) (end 191.580001 71.24208) (width 1) (layer F.Cu) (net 4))
 (segment (start 163.83 71.187919) (end 170.05792 64.959999) (width 1) (layer F.Cu) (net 4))
 (segment (start 163.83 72.39) (end 163.83 71.187919) (width 1) (layer F.Cu) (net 4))
 (segment (start 188.291998 72.39) (end 189.23 72.39) (width 1) (layer F.Cu) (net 4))
 (segment (start 186.69 72.39) (end 189.23 72.39) (width 1) (layer F.Cu) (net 4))
 (segment (start 184.785 74.295) (end 186.69 72.39) (width 1) (layer F.Cu) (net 4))
 (segment (start 163.83 72.39) (end 163.83 76.2) (width 1) (layer F.Cu) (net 4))
 (segment (start 163.83 76.2) (end 167.64 76.2) (width 1) (layer F.Cu) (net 4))
 (segment (start 201.105001 62.419999) (end 200.75501 62.76999) (width 1) (layer F.Cu) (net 9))
 (segment (start 207.875001 62.419999) (end 201.105001 62.419999) (width 1) (layer F.Cu) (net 9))
 (segment (start 208.365001 62.909998) (end 207.875001 62.419999) (width 1) (layer F.Cu) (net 9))
 (segment (start 208.365001 64.77) (end 208.365001 62.909998) (width 1) (layer F.Cu) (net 9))
 (segment (start 161.29 70.54) (end 161.29 72.39) (width 1) (layer F.Cu) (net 9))
 (segment (start 169.06001 62.76999) (end 161.29 70.54) (width 1) (layer F.Cu) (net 9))
 (segment (start 200.75501 62.76999) (end 169.06001 62.76999) (width 1) (layer F.Cu) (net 9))
 (segment (start 190.720522 74.93) (end 194.31 71.340522) (width 1) (layer F.Cu) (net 9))
 (segment (start 189.23 74.93) (end 190.720522 74.93) (width 1) (layer F.Cu) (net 9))
 (segment (start 197.623568 62.76999) (end 200.75501 62.76999) (width 1) (layer F.Cu) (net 9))
 (segment (start 194.31 66.083558) (end 197.623568 62.76999) (width 1) (layer F.Cu) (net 9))
 (segment (start 194.31 71.340522) (end 194.31 66.083558) (width 1) (layer F.Cu) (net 9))
 (segment (start 161.29 76.2) (end 161.29 72.39) (width 1) (layer F.Cu) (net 9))
 (segment (start 203.975001 64.77) (end 205.825001 64.77) (width 1) (layer F.Cu) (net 3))
 (segment (start 198.451998 64.77) (end 203.975001 64.77) (width 1) (layer F.Cu) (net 3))
 (segment (start 197.039999 66.181999) (end 198.451998 64.77) (width 1) (layer F.Cu) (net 3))
 (segment (start 197.039999 73.78208) (end 197.039999 66.181999) (width 1) (layer F.Cu) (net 3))
 (segment (start 198.187919 74.93) (end 197.039999 73.78208) (width 1) (layer F.Cu) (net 3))
 (segment (start 199.39 74.93) (end 198.187919 74.93) (width 1) (layer F.Cu) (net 3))
 (segment (start 188.027919 67.31) (end 189.23 67.31) (width 1) (layer F.Cu) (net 7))
 (segment (start 184.541558 67.31) (end 188.027919 67.31) (width 1) (layer F.Cu) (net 7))
 (segment (start 179.705 72.146558) (end 184.541558 67.31) (width 1) (layer F.Cu) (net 7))
 (segment (start 179.705 74.295) (end 179.705 72.146558) (width 1) (layer F.Cu) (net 7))
 (segment (start 188.003558 69.85) (end 188.027919 69.85) (width 1) (layer F.Cu) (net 8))
 (segment (start 188.027919 69.85) (end 189.23 69.85) (width 1) (layer F.Cu) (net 8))
 (segment (start 184.829998 69.85) (end 188.027919 69.85) (width 1) (layer F.Cu) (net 8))
 (segment (start 182.245 72.434998) (end 184.829998 69.85) (width 1) (layer F.Cu) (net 8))
 (segment (start 182.245 74.295) (end 182.245 72.434998) (width 1) (layer F.Cu) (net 8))
 (segment (start 170.112081 72.39) (end 168.91 72.39) (width 1) (layer F.Cu) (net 10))
 (segment (start 171.27989 72.39) (end 170.112081 72.39) (width 1) (layer F.Cu) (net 10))
 (segment (start 176.35989 77.47) (end 171.27989 72.39) (width 1) (layer F.Cu) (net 10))
 (segment (start 189.23 77.47) (end 176.35989 77.47) (width 1) (layer F.Cu) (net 10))
 (segment (start 199.39 69.85) (end 205.825001 69.85) (width 1) (layer F.Cu) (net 5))
 (segment (start 199.39 67.31) (end 205.825001 67.31) (width 1) (layer F.Cu) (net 6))
 (segment (start 199.39 77.47) (end 205.825001 77.47) (width 1) (layer F.Cu) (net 2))
 (segment (start 205.825001 77.47) (end 208.365001 77.47) (width 1) (layer F.Cu) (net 2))
 (segment (start 173.99 78.16) (end 173.99 78.32499) (width 1) (layer F.Cu) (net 37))
 (segment (start 172.03 76.2) (end 173.99 78.16) (width 1) (layer F.Cu) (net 37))
 (segment (start 170.18 76.2) (end 172.03 76.2) (width 1) (layer F.Cu) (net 37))
 (segment (start 205.825001 80.01) (end 201.740001 80.01) (width 1) (layer F.Cu) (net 15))
 (segment (start 201.740001 80.01) (end 201.740001 82.060001) (width 1) (layer F.Cu) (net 15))
 (segment (start 174.01501 80.42501) (end 173.99 80.42501) (width 1) (layer F.Cu) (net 15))
 (segment (start 175.950001 82.360001) (end 174.01501 80.42501) (width 1) (layer F.Cu) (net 15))
 (segment (start 201.440001 82.360001) (end 175.950001 82.360001) (width 1) (layer F.Cu) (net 15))
 (segment (start 201.740001 82.060001) (end 201.440001 82.360001) (width 1) (layer F.Cu) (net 15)))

